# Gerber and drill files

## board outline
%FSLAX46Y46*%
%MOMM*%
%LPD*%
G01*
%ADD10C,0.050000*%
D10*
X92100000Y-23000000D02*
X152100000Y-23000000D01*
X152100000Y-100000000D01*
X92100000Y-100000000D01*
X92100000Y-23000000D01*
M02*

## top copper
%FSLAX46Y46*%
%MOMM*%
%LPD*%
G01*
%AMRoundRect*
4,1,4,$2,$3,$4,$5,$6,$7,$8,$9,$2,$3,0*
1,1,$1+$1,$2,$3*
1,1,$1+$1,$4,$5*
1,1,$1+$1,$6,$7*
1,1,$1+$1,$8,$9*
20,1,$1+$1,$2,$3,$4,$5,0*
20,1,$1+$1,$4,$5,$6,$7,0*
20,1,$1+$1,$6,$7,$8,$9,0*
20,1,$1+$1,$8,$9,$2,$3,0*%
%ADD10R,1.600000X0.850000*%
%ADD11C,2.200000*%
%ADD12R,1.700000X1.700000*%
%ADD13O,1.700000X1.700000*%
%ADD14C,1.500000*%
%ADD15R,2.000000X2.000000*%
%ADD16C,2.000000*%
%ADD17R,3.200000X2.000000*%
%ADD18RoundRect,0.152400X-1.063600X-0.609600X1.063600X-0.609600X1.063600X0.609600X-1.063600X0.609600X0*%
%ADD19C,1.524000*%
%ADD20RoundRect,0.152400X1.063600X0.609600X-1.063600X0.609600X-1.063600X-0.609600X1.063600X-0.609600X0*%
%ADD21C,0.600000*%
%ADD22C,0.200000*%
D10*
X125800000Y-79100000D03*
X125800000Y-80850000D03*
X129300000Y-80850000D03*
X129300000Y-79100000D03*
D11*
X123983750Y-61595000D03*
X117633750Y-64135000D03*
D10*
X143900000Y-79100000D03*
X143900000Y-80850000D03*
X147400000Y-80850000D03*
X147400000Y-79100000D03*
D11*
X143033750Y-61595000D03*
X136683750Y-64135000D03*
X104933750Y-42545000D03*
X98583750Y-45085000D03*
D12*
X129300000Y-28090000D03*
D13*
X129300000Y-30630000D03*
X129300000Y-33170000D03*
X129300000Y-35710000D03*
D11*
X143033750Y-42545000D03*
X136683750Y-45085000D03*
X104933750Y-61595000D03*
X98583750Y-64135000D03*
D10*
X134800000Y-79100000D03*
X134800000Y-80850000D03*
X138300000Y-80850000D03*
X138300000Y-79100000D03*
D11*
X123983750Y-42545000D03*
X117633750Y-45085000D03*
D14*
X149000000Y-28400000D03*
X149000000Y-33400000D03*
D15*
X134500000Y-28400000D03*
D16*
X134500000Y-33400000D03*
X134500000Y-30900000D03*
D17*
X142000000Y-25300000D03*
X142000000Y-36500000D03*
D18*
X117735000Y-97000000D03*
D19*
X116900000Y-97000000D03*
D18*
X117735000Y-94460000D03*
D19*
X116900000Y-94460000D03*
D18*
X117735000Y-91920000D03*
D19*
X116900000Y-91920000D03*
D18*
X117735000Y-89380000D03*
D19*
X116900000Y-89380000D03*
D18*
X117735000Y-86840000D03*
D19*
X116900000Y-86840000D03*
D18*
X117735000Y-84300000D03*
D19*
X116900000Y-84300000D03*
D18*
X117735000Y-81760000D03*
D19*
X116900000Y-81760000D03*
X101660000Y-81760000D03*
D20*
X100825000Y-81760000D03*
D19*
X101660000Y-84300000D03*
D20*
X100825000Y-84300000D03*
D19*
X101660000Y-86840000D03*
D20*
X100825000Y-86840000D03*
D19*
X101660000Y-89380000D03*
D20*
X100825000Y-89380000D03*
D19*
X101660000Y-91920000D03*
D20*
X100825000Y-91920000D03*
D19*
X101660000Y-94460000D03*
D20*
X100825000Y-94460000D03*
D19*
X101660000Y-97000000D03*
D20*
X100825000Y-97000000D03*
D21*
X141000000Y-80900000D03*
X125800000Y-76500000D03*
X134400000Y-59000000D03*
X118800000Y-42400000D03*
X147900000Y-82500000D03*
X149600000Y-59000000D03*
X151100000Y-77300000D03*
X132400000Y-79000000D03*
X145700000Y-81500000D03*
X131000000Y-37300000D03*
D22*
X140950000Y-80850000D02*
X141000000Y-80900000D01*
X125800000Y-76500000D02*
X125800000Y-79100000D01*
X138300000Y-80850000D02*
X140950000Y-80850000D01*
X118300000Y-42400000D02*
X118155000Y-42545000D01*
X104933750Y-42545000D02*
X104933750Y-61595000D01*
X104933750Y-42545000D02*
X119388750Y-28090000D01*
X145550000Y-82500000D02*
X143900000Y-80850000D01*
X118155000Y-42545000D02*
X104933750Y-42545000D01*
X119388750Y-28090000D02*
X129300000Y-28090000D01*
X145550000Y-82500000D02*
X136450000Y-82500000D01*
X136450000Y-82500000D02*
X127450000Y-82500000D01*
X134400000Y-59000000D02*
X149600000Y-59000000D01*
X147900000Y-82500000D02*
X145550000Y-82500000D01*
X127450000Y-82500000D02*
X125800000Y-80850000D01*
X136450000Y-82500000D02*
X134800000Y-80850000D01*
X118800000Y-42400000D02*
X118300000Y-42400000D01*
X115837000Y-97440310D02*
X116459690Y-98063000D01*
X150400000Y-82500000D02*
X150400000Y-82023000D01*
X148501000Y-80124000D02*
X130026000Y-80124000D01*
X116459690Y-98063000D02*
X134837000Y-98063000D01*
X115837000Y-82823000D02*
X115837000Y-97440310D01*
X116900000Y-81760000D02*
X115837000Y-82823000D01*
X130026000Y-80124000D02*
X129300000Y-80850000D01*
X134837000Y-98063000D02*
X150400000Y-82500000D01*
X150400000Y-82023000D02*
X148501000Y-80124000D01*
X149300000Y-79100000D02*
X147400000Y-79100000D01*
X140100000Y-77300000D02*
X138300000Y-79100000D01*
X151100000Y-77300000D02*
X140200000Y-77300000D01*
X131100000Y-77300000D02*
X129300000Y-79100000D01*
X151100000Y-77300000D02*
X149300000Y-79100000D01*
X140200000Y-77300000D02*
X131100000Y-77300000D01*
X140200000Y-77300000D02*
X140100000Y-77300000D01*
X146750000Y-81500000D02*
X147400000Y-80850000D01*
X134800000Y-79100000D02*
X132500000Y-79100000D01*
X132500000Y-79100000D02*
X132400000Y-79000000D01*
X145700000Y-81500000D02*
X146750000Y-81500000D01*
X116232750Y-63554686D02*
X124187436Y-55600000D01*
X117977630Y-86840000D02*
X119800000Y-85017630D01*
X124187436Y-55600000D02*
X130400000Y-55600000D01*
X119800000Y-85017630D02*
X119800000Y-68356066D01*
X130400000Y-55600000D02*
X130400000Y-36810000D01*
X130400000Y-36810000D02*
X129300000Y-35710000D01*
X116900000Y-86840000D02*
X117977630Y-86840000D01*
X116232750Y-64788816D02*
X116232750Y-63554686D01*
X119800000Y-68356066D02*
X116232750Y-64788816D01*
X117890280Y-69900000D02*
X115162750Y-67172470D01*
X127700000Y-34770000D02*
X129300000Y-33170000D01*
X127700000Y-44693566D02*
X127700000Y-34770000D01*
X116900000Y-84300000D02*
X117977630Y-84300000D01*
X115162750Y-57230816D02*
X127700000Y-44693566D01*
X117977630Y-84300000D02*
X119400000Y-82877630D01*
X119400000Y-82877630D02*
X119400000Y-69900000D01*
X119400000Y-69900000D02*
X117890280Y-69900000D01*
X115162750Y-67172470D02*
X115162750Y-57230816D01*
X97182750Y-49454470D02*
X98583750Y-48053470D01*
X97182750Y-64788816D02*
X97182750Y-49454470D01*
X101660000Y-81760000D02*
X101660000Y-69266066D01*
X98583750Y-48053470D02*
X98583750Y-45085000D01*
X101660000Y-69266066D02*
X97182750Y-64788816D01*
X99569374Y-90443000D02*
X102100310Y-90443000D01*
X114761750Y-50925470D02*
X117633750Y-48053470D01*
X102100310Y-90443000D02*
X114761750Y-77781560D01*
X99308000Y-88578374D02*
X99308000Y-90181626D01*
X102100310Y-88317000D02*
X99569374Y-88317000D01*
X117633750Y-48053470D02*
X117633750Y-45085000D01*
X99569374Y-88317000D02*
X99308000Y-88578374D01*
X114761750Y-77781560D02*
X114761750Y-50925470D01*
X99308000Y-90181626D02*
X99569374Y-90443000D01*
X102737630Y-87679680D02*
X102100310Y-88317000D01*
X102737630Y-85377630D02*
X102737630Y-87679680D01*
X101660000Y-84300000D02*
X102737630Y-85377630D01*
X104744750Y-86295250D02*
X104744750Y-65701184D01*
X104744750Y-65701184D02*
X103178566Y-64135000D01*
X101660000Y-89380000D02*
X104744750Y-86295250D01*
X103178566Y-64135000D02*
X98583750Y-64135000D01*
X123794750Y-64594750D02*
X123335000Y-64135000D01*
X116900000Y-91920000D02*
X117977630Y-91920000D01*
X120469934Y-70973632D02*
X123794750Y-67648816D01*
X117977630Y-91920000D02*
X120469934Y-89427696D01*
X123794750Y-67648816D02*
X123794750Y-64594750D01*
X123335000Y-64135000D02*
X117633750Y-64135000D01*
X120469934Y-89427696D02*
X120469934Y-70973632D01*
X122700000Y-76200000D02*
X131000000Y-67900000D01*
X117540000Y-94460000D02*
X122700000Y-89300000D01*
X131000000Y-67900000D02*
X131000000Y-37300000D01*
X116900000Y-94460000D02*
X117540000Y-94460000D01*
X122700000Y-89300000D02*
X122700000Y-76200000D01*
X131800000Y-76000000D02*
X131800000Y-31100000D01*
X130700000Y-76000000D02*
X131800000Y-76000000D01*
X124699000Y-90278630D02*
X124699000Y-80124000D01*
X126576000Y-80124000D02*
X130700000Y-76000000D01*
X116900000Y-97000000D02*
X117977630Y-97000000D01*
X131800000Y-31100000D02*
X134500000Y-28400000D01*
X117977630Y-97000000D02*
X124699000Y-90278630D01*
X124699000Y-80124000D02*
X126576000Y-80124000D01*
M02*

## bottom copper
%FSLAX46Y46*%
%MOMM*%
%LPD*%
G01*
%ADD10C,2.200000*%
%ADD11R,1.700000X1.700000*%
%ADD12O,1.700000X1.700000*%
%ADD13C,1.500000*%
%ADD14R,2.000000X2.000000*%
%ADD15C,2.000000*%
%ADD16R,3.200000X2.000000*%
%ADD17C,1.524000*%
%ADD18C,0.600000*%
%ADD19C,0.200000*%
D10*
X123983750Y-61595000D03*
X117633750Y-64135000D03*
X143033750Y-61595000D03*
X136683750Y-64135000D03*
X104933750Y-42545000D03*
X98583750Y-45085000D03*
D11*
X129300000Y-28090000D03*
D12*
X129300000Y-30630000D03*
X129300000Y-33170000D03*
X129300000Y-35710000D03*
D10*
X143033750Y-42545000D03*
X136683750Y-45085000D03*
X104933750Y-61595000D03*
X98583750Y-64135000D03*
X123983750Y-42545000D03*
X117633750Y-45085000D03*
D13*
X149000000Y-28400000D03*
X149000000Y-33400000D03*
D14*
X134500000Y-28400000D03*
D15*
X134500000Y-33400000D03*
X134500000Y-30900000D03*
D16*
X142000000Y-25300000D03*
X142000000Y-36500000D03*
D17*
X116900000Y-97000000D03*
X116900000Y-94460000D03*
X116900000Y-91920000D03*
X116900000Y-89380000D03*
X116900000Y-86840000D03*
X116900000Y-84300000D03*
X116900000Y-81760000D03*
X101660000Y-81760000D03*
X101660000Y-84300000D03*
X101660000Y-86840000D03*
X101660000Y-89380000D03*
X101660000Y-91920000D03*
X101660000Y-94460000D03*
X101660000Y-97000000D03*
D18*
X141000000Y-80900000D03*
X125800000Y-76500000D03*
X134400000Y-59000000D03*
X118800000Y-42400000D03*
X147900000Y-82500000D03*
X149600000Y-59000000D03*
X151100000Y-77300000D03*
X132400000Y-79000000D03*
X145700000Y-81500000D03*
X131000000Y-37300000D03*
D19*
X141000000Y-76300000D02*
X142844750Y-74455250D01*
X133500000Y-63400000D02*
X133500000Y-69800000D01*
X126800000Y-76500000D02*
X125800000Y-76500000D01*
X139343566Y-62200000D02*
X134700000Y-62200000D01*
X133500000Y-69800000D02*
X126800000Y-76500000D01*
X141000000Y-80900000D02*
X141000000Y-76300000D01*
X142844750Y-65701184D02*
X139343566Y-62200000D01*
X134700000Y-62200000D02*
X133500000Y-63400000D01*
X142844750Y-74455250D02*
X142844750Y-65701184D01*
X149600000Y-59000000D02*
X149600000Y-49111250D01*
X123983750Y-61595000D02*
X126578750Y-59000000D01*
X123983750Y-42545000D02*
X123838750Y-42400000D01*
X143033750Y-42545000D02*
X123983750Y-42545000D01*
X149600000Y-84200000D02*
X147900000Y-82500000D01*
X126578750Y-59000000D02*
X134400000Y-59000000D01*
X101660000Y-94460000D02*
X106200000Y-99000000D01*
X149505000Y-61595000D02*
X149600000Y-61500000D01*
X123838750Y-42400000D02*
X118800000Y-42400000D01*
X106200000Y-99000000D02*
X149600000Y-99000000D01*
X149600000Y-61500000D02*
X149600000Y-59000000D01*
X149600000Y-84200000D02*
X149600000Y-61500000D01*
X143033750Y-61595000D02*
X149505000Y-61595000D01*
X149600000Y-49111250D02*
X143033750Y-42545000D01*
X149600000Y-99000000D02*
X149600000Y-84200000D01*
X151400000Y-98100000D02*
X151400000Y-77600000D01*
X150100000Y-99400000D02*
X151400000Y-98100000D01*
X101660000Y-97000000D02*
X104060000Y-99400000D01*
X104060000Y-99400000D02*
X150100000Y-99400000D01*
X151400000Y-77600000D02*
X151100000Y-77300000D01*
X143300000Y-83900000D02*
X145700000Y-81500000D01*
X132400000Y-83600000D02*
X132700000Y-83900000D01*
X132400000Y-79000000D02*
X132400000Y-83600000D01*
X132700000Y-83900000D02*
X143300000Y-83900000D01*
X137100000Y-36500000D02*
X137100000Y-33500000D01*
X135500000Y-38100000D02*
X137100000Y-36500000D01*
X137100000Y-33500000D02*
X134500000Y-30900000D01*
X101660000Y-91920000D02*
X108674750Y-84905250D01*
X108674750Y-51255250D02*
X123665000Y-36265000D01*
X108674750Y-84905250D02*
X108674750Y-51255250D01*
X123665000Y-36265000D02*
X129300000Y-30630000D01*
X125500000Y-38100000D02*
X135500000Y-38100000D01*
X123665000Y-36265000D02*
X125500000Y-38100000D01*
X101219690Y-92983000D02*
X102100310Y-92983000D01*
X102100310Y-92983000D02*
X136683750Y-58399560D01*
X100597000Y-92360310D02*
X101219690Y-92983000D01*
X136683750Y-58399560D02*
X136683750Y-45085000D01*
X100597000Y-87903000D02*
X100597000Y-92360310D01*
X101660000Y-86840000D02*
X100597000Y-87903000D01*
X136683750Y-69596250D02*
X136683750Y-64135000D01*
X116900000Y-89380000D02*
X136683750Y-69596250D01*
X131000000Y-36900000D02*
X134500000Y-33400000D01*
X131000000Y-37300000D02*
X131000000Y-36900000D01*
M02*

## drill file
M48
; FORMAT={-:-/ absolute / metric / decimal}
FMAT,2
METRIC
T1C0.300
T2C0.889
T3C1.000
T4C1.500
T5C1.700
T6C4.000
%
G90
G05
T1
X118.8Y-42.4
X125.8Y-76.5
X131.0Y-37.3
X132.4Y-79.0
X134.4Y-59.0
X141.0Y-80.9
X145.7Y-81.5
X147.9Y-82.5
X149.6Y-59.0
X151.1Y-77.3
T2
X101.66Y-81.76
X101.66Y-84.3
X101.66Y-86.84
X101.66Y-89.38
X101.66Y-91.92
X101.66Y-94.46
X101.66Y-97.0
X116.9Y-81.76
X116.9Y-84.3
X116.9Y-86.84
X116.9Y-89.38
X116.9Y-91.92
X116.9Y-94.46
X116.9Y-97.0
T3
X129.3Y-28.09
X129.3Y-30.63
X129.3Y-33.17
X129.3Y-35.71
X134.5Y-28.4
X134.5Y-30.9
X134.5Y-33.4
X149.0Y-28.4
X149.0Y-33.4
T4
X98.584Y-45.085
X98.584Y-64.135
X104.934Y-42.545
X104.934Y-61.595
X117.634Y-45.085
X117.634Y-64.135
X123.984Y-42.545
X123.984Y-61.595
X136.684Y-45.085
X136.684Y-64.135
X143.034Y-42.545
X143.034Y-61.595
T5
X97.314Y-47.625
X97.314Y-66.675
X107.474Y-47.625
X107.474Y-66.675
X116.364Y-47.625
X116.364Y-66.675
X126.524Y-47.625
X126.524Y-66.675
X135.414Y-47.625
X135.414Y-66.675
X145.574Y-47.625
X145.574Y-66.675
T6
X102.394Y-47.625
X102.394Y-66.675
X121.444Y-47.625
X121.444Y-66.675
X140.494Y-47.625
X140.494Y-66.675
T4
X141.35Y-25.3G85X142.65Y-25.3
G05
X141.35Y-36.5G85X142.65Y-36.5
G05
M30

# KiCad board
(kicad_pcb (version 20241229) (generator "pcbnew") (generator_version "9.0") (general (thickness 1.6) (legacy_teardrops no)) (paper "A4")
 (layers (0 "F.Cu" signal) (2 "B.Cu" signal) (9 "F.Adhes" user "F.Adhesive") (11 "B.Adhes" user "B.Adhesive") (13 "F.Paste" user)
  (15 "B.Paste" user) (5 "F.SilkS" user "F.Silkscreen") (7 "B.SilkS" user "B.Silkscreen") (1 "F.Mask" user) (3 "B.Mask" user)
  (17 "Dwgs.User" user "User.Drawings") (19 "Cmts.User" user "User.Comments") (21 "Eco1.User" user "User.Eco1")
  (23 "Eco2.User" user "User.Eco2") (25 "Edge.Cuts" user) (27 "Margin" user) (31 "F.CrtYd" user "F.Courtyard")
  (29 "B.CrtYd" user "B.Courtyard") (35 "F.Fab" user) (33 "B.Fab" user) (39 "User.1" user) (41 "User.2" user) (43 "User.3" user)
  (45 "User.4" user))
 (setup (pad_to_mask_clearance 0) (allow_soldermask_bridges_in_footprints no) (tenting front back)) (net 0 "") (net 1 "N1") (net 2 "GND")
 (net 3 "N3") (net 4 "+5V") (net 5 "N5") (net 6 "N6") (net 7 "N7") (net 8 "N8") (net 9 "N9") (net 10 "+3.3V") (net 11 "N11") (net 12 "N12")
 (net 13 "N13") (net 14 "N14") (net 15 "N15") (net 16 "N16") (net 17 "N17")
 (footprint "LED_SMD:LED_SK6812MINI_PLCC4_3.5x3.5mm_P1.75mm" (layer "F.Cu") (at 127.55 79.975)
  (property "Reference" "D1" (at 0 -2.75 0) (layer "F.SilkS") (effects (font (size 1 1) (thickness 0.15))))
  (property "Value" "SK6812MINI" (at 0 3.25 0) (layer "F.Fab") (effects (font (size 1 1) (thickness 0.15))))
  (pad "1" smd rect (at -1.75 -0.875) (size 1.6 0.85) (layers "F.Cu" "F.Mask" "F.Paste") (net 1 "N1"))
  (pad "2" smd rect (at -1.75 0.875) (size 1.6 0.85) (layers "F.Cu" "F.Mask" "F.Paste") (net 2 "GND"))
  (pad "3" smd rect (at 1.75 0.875) (size 1.6 0.85) (layers "F.Cu" "F.Mask" "F.Paste") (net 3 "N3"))
  (pad "4" smd rect (at 1.75 -0.875) (size 1.6 0.85) (layers "F.Cu" "F.Mask" "F.Paste") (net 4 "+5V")))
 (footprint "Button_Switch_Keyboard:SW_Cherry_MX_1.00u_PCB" (layer "F.Cu") (at 123.98375 61.595)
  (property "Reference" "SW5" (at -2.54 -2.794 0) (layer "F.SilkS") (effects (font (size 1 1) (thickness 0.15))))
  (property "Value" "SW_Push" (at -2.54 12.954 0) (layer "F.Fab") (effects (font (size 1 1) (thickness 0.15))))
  (pad "" np_thru_hole circle (at -7.62 5.08) (size 1.7 1.7) (drill 1.7) (layers "*.Cu" "*.Mask"))
  (pad "" np_thru_hole circle (at -2.54 5.08) (size 4 4) (drill 4) (layers "*.Cu" "*.Mask"))
  (pad "" np_thru_hole circle (at 2.54 5.08) (size 1.7 1.7) (drill 1.7) (layers "*.Cu" "*.Mask"))
  (pad "1" thru_hole circle (at 0 0) (size 2.2 2.2) (drill 1.5) (layers "*.Cu" "*.Mask") (remove_unused_layers no) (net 2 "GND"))
  (pad "2" thru_hole circle (at -6.35 2.54) (size 2.2 2.2) (drill 1.5) (layers "*.Cu" "*.Mask") (remove_unused_layers no) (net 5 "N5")))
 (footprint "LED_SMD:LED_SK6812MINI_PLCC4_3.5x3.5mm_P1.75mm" (layer "F.Cu") (at 145.65 79.975)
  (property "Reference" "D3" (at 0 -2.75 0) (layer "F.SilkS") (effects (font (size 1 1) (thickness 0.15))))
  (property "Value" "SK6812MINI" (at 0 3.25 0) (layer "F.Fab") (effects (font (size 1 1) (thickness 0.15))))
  (pad "1" smd rect (at -1.75 -0.875) (size 1.6 0.85) (layers "F.Cu" "F.Mask" "F.Paste") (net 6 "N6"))
  (pad "2" smd rect (at -1.75 0.875) (size 1.6 0.85) (layers "F.Cu" "F.Mask" "F.Paste") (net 2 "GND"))
  (pad "3" smd rect (at 1.75 0.875) (size 1.6 0.85) (layers "F.Cu" "F.Mask" "F.Paste") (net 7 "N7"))
  (pad "4" smd rect (at 1.75 -0.875) (size 1.6 0.85) (layers "F.Cu" "F.Mask" "F.Paste") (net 4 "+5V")))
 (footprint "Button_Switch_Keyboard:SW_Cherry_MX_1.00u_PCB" (layer "F.Cu") (at 143.03375 61.595)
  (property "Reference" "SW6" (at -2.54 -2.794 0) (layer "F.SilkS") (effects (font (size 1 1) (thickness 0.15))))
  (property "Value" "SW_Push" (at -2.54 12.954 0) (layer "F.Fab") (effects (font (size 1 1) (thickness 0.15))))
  (pad "" np_thru_hole circle (at -7.62 5.08) (size 1.7 1.7) (drill 1.7) (layers "*.Cu" "*.Mask"))
  (pad "" np_thru_hole circle (at -2.54 5.08) (size 4 4) (drill 4) (layers "*.Cu" "*.Mask"))
  (pad "" np_thru_hole circle (at 2.54 5.08) (size 1.7 1.7) (drill 1.7) (layers "*.Cu" "*.Mask"))
  (pad "1" thru_hole circle (at 0 0) (size 2.2 2.2) (drill 1.5) (layers "*.Cu" "*.Mask") (remove_unused_layers no) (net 2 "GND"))
  (pad "2" thru_hole circle (at -6.35 2.54) (size 2.2 2.2) (drill 1.5) (layers "*.Cu" "*.Mask") (remove_unused_layers no) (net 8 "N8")))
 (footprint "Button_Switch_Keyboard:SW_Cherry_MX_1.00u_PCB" (layer "F.Cu") (at 104.93375 42.545)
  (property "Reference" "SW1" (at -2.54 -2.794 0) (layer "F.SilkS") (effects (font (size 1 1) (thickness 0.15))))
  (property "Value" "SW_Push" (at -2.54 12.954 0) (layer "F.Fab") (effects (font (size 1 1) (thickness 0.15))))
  (pad "" np_thru_hole circle (at -7.62 5.08) (size 1.7 1.7) (drill 1.7) (layers "*.Cu" "*.Mask"))
  (pad "" np_thru_hole circle (at -2.54 5.08) (size 4 4) (drill 4) (layers "*.Cu" "*.Mask"))
  (pad "" np_thru_hole circle (at 2.54 5.08) (size 1.7 1.7) (drill 1.7) (layers "*.Cu" "*.Mask"))
  (pad "1" thru_hole circle (at 0 0) (size 2.2 2.2) (drill 1.5) (layers "*.Cu" "*.Mask") (remove_unused_layers no) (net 2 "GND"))
  (pad "2" thru_hole circle (at -6.35 2.54) (size 2.2 2.2) (drill 1.5) (layers "*.Cu" "*.Mask") (remove_unused_layers no) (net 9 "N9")))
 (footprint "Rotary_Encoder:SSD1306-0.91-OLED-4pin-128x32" (layer "F.Cu") (at 92.8 25.9)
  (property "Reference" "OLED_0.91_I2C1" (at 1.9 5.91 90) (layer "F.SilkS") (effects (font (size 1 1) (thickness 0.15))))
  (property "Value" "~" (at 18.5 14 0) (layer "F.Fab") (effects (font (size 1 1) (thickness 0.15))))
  (pad "1" thru_hole rect (at 36.5 2.19) (size 1.7 1.7) (drill 1) (layers "*.Cu" "*.Mask") (remove_unused_layers no) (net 2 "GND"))
  (pad "2" thru_hole oval (at 36.5 4.73) (size 1.7 1.7) (drill 1) (layers "*.Cu" "*.Mask") (remove_unused_layers no) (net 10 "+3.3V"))
  (pad "3" thru_hole oval (at 36.5 7.27) (size 1.7 1.7) (drill 1) (layers "*.Cu" "*.Mask") (remove_unused_layers no) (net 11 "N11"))
  (pad "4" thru_hole oval (at 36.5 9.81) (size 1.7 1.7) (drill 1) (layers "*.Cu" "*.Mask") (remove_unused_layers no) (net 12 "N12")))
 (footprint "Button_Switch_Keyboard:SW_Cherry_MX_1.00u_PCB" (layer "F.Cu") (at 143.03375 42.545)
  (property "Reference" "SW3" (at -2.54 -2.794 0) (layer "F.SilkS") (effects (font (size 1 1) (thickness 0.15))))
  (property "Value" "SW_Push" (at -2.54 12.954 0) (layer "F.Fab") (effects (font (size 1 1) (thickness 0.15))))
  (pad "" np_thru_hole circle (at -7.62 5.08) (size 1.7 1.7) (drill 1.7) (layers "*.Cu" "*.Mask"))
  (pad "" np_thru_hole circle (at -2.54 5.08) (size 4 4) (drill 4) (layers "*.Cu" "*.Mask"))
  (pad "" np_thru_hole circle (at 2.54 5.08) (size 1.7 1.7) (drill 1.7) (layers "*.Cu" "*.Mask"))
  (pad "1" thru_hole circle (at 0 0) (size 2.2 2.2) (drill 1.5) (layers "*.Cu" "*.Mask") (remove_unused_layers no) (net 2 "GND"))
  (pad "2" thru_hole circle (at -6.35 2.54) (size 2.2 2.2) (drill 1.5) (layers "*.Cu" "*.Mask") (remove_unused_layers no) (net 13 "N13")))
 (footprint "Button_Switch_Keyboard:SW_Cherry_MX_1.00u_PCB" (layer "F.Cu") (at 104.93375 61.595)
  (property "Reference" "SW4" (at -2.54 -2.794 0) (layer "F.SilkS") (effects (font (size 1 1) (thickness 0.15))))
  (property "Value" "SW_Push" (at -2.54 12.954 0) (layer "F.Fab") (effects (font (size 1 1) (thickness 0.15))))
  (pad "" np_thru_hole circle (at -7.62 5.08) (size 1.7 1.7) (drill 1.7) (layers "*.Cu" "*.Mask"))
  (pad "" np_thru_hole circle (at -2.54 5.08) (size 4 4) (drill 4) (layers "*.Cu" "*.Mask"))
  (pad "" np_thru_hole circle (at 2.54 5.08) (size 1.7 1.7) (drill 1.7) (layers "*.Cu" "*.Mask"))
  (pad "1" thru_hole circle (at 0 0) (size 2.2 2.2) (drill 1.5) (layers "*.Cu" "*.Mask") (remove_unused_layers no) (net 2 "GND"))
  (pad "2" thru_hole circle (at -6.35 2.54) (size 2.2 2.2) (drill 1.5) (layers "*.Cu" "*.Mask") (remove_unused_layers no) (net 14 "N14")))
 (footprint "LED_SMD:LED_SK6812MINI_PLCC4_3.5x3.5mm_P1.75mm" (layer "F.Cu") (at 136.55 79.975)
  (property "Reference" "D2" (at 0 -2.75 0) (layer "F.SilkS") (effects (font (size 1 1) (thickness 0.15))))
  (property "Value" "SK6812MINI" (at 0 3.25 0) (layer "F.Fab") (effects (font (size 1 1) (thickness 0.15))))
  (pad "1" smd rect (at -1.75 -0.875) (size 1.6 0.85) (layers "F.Cu" "F.Mask" "F.Paste") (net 7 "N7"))
  (pad "2" smd rect (at -1.75 0.875) (size 1.6 0.85) (layers "F.Cu" "F.Mask" "F.Paste") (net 2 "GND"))
  (pad "3" smd rect (at 1.75 0.875) (size 1.6 0.85) (layers "F.Cu" "F.Mask" "F.Paste") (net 1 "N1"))
  (pad "4" smd rect (at 1.75 -0.875) (size 1.6 0.85) (layers "F.Cu" "F.Mask" "F.Paste") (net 4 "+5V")))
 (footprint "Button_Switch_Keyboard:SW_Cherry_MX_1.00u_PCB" (layer "F.Cu") (at 123.98375 42.545)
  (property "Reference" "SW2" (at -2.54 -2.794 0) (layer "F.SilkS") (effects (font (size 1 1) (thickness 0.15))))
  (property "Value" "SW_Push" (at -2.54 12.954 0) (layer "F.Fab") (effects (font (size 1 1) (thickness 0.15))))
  (pad "" np_thru_hole circle (at -7.62 5.08) (size 1.7 1.7) (drill 1.7) (layers "*.Cu" "*.Mask"))
  (pad "" np_thru_hole circle (at -2.54 5.08) (size 4 4) (drill 4) (layers "*.Cu" "*.Mask"))
  (pad "" np_thru_hole circle (at 2.54 5.08) (size 1.7 1.7) (drill 1.7) (layers "*.Cu" "*.Mask"))
  (pad "1" thru_hole circle (at 0 0) (size 2.2 2.2) (drill 1.5) (layers "*.Cu" "*.Mask") (remove_unused_layers no) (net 2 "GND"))
  (pad "2" thru_hole circle (at -6.35 2.54) (size 2.2 2.2) (drill 1.5) (layers "*.Cu" "*.Mask") (remove_unused_layers no) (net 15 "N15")))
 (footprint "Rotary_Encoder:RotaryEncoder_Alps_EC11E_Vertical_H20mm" (layer "F.Cu") (at 134.5 28.4)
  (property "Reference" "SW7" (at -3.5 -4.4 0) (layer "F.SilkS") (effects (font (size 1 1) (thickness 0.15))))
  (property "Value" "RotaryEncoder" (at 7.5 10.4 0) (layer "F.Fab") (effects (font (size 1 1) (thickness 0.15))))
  (pad "" thru_hole circle (at 14.5 0) (size 1.5 1.5) (drill 1) (layers "*.Cu" "*.Mask") (remove_unused_layers no))
  (pad "" thru_hole circle (at 14.5 5) (size 1.5 1.5) (drill 1) (layers "*.Cu" "*.Mask") (remove_unused_layers no))
  (pad "A" thru_hole rect (at 0 0) (size 2 2) (drill 1) (layers "*.Cu" "*.Mask") (remove_unused_layers no) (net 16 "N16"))
  (pad "B" thru_hole circle (at 0 5) (size 2 2) (drill 1) (layers "*.Cu" "*.Mask") (remove_unused_layers no) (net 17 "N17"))
  (pad "C" thru_hole circle (at 0 2.5) (size 2 2) (drill 1) (layers "*.Cu" "*.Mask") (remove_unused_layers no) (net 10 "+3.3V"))
  (pad "MP" thru_hole rect (at 7.5 -3.1) (size 3.2 2) (drill oval 2.8 1.5) (layers "*.Cu" "*.Mask") (remove_unused_layers no))
  (pad "MP" thru_hole rect (at 7.5 8.1) (size 3.2 2) (drill oval 2.8 1.5) (layers "*.Cu" "*.Mask") (remove_unused_layers no)))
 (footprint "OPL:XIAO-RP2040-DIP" (layer "F.Cu") (at 109.28 89.38 180)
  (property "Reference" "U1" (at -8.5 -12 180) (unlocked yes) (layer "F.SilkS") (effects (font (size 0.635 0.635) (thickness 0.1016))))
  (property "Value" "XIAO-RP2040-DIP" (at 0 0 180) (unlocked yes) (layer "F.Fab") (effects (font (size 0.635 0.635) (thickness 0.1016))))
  (pad "1" smd roundrect (at -8.455 -7.62) (size 2.432 1.524) (layers "F.Cu" "F.Mask") (roundrect_rratio 0.1) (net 16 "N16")
   (thermal_bridge_angle 45))
  (pad "1" thru_hole circle (at -7.62 -7.62) (size 1.524 1.524) (drill 0.889) (layers "*.Cu" "*.Mask") (remove_unused_layers no)
   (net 16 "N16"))
  (pad "2" smd roundrect (at -8.455 -5.08) (size 2.432 1.524) (layers "F.Cu" "F.Mask") (roundrect_rratio 0.1) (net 17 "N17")
   (thermal_bridge_angle 45))
  (pad "2" thru_hole circle (at -7.62 -5.08) (size 1.524 1.524) (drill 0.889) (layers "*.Cu" "*.Mask") (remove_unused_layers no)
   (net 17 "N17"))
  (pad "3" smd roundrect (at -8.455 -2.54) (size 2.432 1.524) (layers "F.Cu" "F.Mask") (roundrect_rratio 0.1) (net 5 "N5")
   (thermal_bridge_angle 45))
  (pad "3" thru_hole circle (at -7.62 -2.54) (size 1.524 1.524) (drill 0.889) (layers "*.Cu" "*.Mask") (remove_unused_layers no)
   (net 5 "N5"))
  (pad "4" smd roundrect (at -8.455 0) (size 2.432 1.524) (layers "F.Cu" "F.Mask") (roundrect_rratio 0.1) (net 8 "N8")
   (thermal_bridge_angle 45))
  (pad "4" thru_hole circle (at -7.62 0) (size 1.524 1.524) (drill 0.889) (layers "*.Cu" "*.Mask") (remove_unused_layers no) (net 8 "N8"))
  (pad "5" smd roundrect (at -8.455 2.54) (size 2.432 1.524) (layers "F.Cu" "F.Mask") (roundrect_rratio 0.1) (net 12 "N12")
   (thermal_bridge_angle 45))
  (pad "5" thru_hole circle (at -7.62 2.54) (size 1.524 1.524) (drill 0.889) (layers "*.Cu" "*.Mask") (remove_unused_layers no)
   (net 12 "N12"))
  (pad "6" smd roundrect (at -8.455 5.08) (size 2.432 1.524) (layers "F.Cu" "F.Mask") (roundrect_rratio 0.1) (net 11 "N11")
   (thermal_bridge_angle 45))
  (pad "6" thru_hole circle (at -7.62 5.08) (size 1.524 1.524) (drill 0.889) (layers "*.Cu" "*.Mask") (remove_unused_layers no)
   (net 11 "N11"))
  (pad "7" smd roundrect (at -8.455 7.62) (size 2.432 1.524) (layers "F.Cu" "F.Mask") (roundrect_rratio 0.1) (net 3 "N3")
   (thermal_bridge_angle 45))
  (pad "7" thru_hole circle (at -7.62 7.62) (size 1.524 1.524) (drill 0.889) (layers "*.Cu" "*.Mask") (remove_unused_layers no) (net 3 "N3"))
  (pad "8" thru_hole circle (at 7.62 7.62 180) (size 1.524 1.524) (drill 0.889) (layers "*.Cu" "*.Mask") (remove_unused_layers no)
   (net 9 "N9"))
  (pad "8" smd roundrect (at 8.455 7.62 180) (size 2.432 1.524) (layers "F.Cu" "F.Mask") (roundrect_rratio 0.1) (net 9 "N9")
   (thermal_bridge_angle 45))
  (pad "9" thru_hole circle (at 7.62 5.08 180) (size 1.524 1.524) (drill 0.889) (layers "*.Cu" "*.Mask") (remove_unused_layers no)
   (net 15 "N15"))
  (pad "9" smd roundrect (at 8.455 5.08 180) (size 2.432 1.524) (layers "F.Cu" "F.Mask") (roundrect_rratio 0.1) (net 15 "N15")
   (thermal_bridge_angle 45))
  (pad "10" thru_hole circle (at 7.62 2.54 180) (size 1.524 1.524) (drill 0.889) (layers "*.Cu" "*.Mask") (remove_unused_layers no)
   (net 13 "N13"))
  (pad "10" smd roundrect (at 8.455 2.54 180) (size 2.432 1.524) (layers "F.Cu" "F.Mask") (roundrect_rratio 0.1) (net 13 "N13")
   (thermal_bridge_angle 45))
  (pad "11" thru_hole circle (at 7.62 0 180) (size 1.524 1.524) (drill 0.889) (layers "*.Cu" "*.Mask") (remove_unused_layers no)
   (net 14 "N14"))
  (pad "11" smd roundrect (at 8.455 0 180) (size 2.432 1.524) (layers "F.Cu" "F.Mask") (roundrect_rratio 0.1) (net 14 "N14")
   (thermal_bridge_angle 45))
  (pad "12" thru_hole circle (at 7.62 -2.54 180) (size 1.524 1.524) (drill 0.889) (layers "*.Cu" "*.Mask") (remove_unused_layers no)
   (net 10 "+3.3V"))
  (pad "12" smd roundrect (at 8.455 -2.54 180) (size 2.432 1.524) (layers "F.Cu" "F.Mask") (roundrect_rratio 0.1) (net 10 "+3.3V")
   (thermal_bridge_angle 45))
  (pad "13" thru_hole circle (at 7.62 -5.08 180) (size 1.524 1.524) (drill 0.889) (layers "*.Cu" "*.Mask") (remove_unused_layers no)
   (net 2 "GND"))
  (pad "13" smd roundrect (at 8.455 -5.08 180) (size 2.432 1.524) (layers "F.Cu" "F.Mask") (roundrect_rratio 0.1) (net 2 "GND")
   (thermal_bridge_angle 45))
  (pad "14" thru_hole circle (at 7.62 -7.62 180) (size 1.524 1.524) (drill 0.889) (layers "*.Cu" "*.Mask") (remove_unused_layers no)
   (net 4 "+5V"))
  (pad "14" smd roundrect (at 8.455 -7.62 180) (size 2.432 1.524) (layers "F.Cu" "F.Mask") (roundrect_rratio 0.1) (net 4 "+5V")
   (thermal_bridge_angle 45)))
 (gr_rect (start 92.1 23) (end 152.1 100) (stroke (width 0.05) (type default)) (fill no) (layer "Edge.Cuts"))
 (segment (start 140.95 80.85) (end 141 80.9) (width 0.2) (layer "F.Cu") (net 1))
 (segment (start 125.8 76.5) (end 125.8 79.1) (width 0.2) (layer "F.Cu") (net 1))
 (segment (start 138.3 80.85) (end 140.95 80.85) (width 0.2) (layer "F.Cu") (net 1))
 (via (at 141 80.9) (size 0.6) (drill 0.3) (layers "F.Cu" "B.Cu") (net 1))
 (via (at 125.8 76.5) (size 0.6) (drill 0.3) (layers "F.Cu" "B.Cu") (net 1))
 (segment (start 141 76.3) (end 142.84475 74.45525) (width 0.2) (layer "B.Cu") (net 1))
 (segment (start 133.5 63.4) (end 133.5 69.8) (width 0.2) (layer "B.Cu") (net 1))
 (segment (start 126.8 76.5) (end 125.8 76.5) (width 0.2) (layer "B.Cu") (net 1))
 (segment (start 139.343566 62.2) (end 134.7 62.2) (width 0.2) (layer "B.Cu") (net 1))
 (segment (start 133.5 69.8) (end 126.8 76.5) (width 0.2) (layer "B.Cu") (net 1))
 (segment (start 141 80.9) (end 141 76.3) (width 0.2) (layer "B.Cu") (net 1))
 (segment (start 142.84475 65.701184) (end 139.343566 62.2) (width 0.2) (layer "B.Cu") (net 1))
 (segment (start 134.7 62.2) (end 133.5 63.4) (width 0.2) (layer "B.Cu") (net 1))
 (segment (start 142.84475 74.45525) (end 142.84475 65.701184) (width 0.2) (layer "B.Cu") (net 1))
 (segment (start 118.3 42.4) (end 118.155 42.545) (width 0.2) (layer "F.Cu") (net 2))
 (segment (start 104.93375 42.545) (end 104.93375 61.595) (width 0.2) (layer "F.Cu") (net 2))
 (segment (start 104.93375 42.545) (end 119.38875 28.09) (width 0.2) (layer "F.Cu") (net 2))
 (segment (start 145.55 82.5) (end 143.9 80.85) (width 0.2) (layer "F.Cu") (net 2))
 (segment (start 118.155 42.545) (end 104.93375 42.545) (width 0.2) (layer "F.Cu") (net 2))
 (segment (start 119.38875 28.09) (end 129.3 28.09) (width 0.2) (layer "F.Cu") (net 2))
 (segment (start 145.55 82.5) (end 136.45 82.5) (width 0.2) (layer "F.Cu") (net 2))
 (segment (start 136.45 82.5) (end 127.45 82.5) (width 0.2) (layer "F.Cu") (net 2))
 (segment (start 134.4 59) (end 149.6 59) (width 0.2) (layer "F.Cu") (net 2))
 (segment (start 147.9 82.5) (end 145.55 82.5) (width 0.2) (layer "F.Cu") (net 2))
 (segment (start 127.45 82.5) (end 125.8 80.85) (width 0.2) (layer "F.Cu") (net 2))
 (segment (start 136.45 82.5) (end 134.8 80.85) (width 0.2) (layer "F.Cu") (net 2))
 (segment (start 118.8 42.4) (end 118.3 42.4) (width 0.2) (layer "F.Cu") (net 2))
 (via (at 134.4 59) (size 0.6) (drill 0.3) (layers "F.Cu" "B.Cu") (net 2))
 (via (at 118.8 42.4) (size 0.6) (drill 0.3) (layers "F.Cu" "B.Cu") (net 2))
 (via (at 147.9 82.5) (size 0.6) (drill 0.3) (layers "F.Cu" "B.Cu") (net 2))
 (via (at 149.6 59) (size 0.6) (drill 0.3) (layers "F.Cu" "B.Cu") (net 2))
 (segment (start 149.6 59) (end 149.6 49.11125) (width 0.2) (layer "B.Cu") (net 2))
 (segment (start 123.98375 61.595) (end 126.57875 59) (width 0.2) (layer "B.Cu") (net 2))
 (segment (start 123.98375 42.545) (end 123.83875 42.4) (width 0.2) (layer "B.Cu") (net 2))
 (segment (start 143.03375 42.545) (end 123.98375 42.545) (width 0.2) (layer "B.Cu") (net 2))
 (segment (start 149.6 84.2) (end 147.9 82.5) (width 0.2) (layer "B.Cu") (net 2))
 (segment (start 126.57875 59) (end 134.4 59) (width 0.2) (layer "B.Cu") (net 2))
 (segment (start 101.66 94.46) (end 106.2 99) (width 0.2) (layer "B.Cu") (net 2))
 (segment (start 149.505 61.595) (end 149.6 61.5) (width 0.2) (layer "B.Cu") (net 2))
 (segment (start 123.83875 42.4) (end 118.8 42.4) (width 0.2) (layer "B.Cu") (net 2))
 (segment (start 106.2 99) (end 149.6 99) (width 0.2) (layer "B.Cu") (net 2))
 (segment (start 149.6 61.5) (end 149.6 59) (width 0.2) (layer "B.Cu") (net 2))
 (segment (start 149.6 84.2) (end 149.6 61.5) (width 0.2) (layer "B.Cu") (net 2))
 (segment (start 143.03375 61.595) (end 149.505 61.595) (width 0.2) (layer "B.Cu") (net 2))
 (segment (start 149.6 49.11125) (end 143.03375 42.545) (width 0.2) (layer "B.Cu") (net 2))
 (segment (start 149.6 99) (end 149.6 84.2) (width 0.2) (layer "B.Cu") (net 2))
 (segment (start 115.837 97.44031) (end 116.45969 98.063) (width 0.2) (layer "F.Cu") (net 3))
 (segment (start 150.4 82.5) (end 150.4 82.023) (width 0.2) (layer "F.Cu") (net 3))
 (segment (start 148.501 80.124) (end 130.026 80.124) (width 0.2) (layer "F.Cu") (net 3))
 (segment (start 116.45969 98.063) (end 134.837 98.063) (width 0.2) (layer "F.Cu") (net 3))
 (segment (start 115.837 82.823) (end 115.837 97.44031) (width 0.2) (layer "F.Cu") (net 3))
 (segment (start 116.9 81.76) (end 115.837 82.823) (width 0.2) (layer "F.Cu") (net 3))
 (segment (start 130.026 80.124) (end 129.3 80.85) (width 0.2) (layer "F.Cu") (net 3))
 (segment (start 134.837 98.063) (end 150.4 82.5) (width 0.2) (layer "F.Cu") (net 3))
 (segment (start 150.4 82.023) (end 148.501 80.124) (width 0.2) (layer "F.Cu") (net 3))
 (segment (start 149.3 79.1) (end 147.4 79.1) (width 0.2) (layer "F.Cu") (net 4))
 (segment (start 140.1 77.3) (end 138.3 79.1) (width 0.2) (layer "F.Cu") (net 4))
 (segment (start 151.1 77.3) (end 140.2 77.3) (width 0.2) (layer "F.Cu") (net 4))
 (segment (start 131.1 77.3) (end 129.3 79.1) (width 0.2) (layer "F.Cu") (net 4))
 (segment (start 151.1 77.3) (end 149.3 79.1) (width 0.2) (layer "F.Cu") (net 4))
 (segment (start 140.2 77.3) (end 131.1 77.3) (width 0.2) (layer "F.Cu") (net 4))
 (segment (start 140.2 77.3) (end 140.1 77.3) (width 0.2) (layer "F.Cu") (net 4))
 (via (at 151.1 77.3) (size 0.6) (drill 0.3) (layers "F.Cu" "B.Cu") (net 4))
 (segment (start 151.4 98.1) (end 151.4 77.6) (width 0.2) (layer "B.Cu") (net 4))
 (segment (start 150.1 99.4) (end 151.4 98.1) (width 0.2) (layer "B.Cu") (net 4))
 (segment (start 101.66 97) (end 104.06 99.4) (width 0.2) (layer "B.Cu") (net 4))
 (segment (start 104.06 99.4) (end 150.1 99.4) (width 0.2) (layer "B.Cu") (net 4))
 (segment (start 151.4 77.6) (end 151.1 77.3) (width 0.2) (layer "B.Cu") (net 4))
 (segment (start 146.75 81.5) (end 147.4 80.85) (width 0.2) (layer "F.Cu") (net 7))
 (segment (start 134.8 79.1) (end 132.5 79.1) (width 0.2) (layer "F.Cu") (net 7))
 (segment (start 132.5 79.1) (end 132.4 79) (width 0.2) (layer "F.Cu") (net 7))
 (segment (start 145.7 81.5) (end 146.75 81.5) (width 0.2) (layer "F.Cu") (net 7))
 (via (at 132.4 79) (size 0.6) (drill 0.3) (layers "F.Cu" "B.Cu") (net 7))
 (via (at 145.7 81.5) (size 0.6) (drill 0.3) (layers "F.Cu" "B.Cu") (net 7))
 (segment (start 143.3 83.9) (end 145.7 81.5) (width 0.2) (layer "B.Cu") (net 7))
 (segment (start 132.4 83.6) (end 132.7 83.9) (width 0.2) (layer "B.Cu") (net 7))
 (segment (start 132.4 79) (end 132.4 83.6) (width 0.2) (layer "B.Cu") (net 7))
 (segment (start 132.7 83.9) (end 143.3 83.9) (width 0.2) (layer "B.Cu") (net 7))
 (segment (start 137.1 36.5) (end 137.1 33.5) (width 0.2) (layer "B.Cu") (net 10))
 (segment (start 135.5 38.1) (end 137.1 36.5) (width 0.2) (layer "B.Cu") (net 10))
 (segment (start 137.1 33.5) (end 134.5 30.9) (width 0.2) (layer "B.Cu") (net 10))
 (segment (start 101.66 91.92) (end 108.67475 84.90525) (width 0.2) (layer "B.Cu") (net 10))
 (segment (start 108.67475 51.25525) (end 123.665 36.265) (width 0.2) (layer "B.Cu") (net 10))
 (segment (start 108.67475 84.90525) (end 108.67475 51.25525) (width 0.2) (layer "B.Cu") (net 10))
 (segment (start 123.665 36.265) (end 129.3 30.63) (width 0.2) (layer "B.Cu") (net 10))
 (segment (start 125.5 38.1) (end 135.5 38.1) (width 0.2) (layer "B.Cu") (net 10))
 (segment (start 123.665 36.265) (end 125.5 38.1) (width 0.2) (layer "B.Cu") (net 10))
 (segment (start 116.23275 63.554686) (end 124.187436 55.6) (width 0.2) (layer "F.Cu") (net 12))
 (segment (start 117.97763 86.84) (end 119.8 85.01763) (width 0.2) (layer "F.Cu") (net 12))
 (segment (start 124.187436 55.6) (end 130.4 55.6) (width 0.2) (layer "F.Cu") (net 12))
 (segment (start 119.8 85.01763) (end 119.8 68.356066) (width 0.2) (layer "F.Cu") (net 12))
 (segment (start 130.4 55.6) (end 130.4 36.81) (width 0.2) (layer "F.Cu") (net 12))
 (segment (start 130.4 36.81) (end 129.3 35.71) (width 0.2) (layer "F.Cu") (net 12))
 (segment (start 116.9 86.84) (end 117.97763 86.84) (width 0.2) (layer "F.Cu") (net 12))
 (segment (start 116.23275 64.788816) (end 116.23275 63.554686) (width 0.2) (layer "F.Cu") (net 12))
 (segment (start 119.8 68.356066) (end 116.23275 64.788816) (width 0.2) (layer "F.Cu") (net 12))
 (segment (start 117.89028 69.9) (end 115.16275 67.17247) (width 0.2) (layer "F.Cu") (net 11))
 (segment (start 127.7 34.77) (end 129.3 33.17) (width 0.2) (layer "F.Cu") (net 11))
 (segment (start 127.7 44.693566) (end 127.7 34.77) (width 0.2) (layer "F.Cu") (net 11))
 (segment (start 116.9 84.3) (end 117.97763 84.3) (width 0.2) (layer "F.Cu") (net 11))
 (segment (start 115.16275 57.230816) (end 127.7 44.693566) (width 0.2) (layer "F.Cu") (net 11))
 (segment (start 117.97763 84.3) (end 119.4 82.87763) (width 0.2) (layer "F.Cu") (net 11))
 (segment (start 119.4 82.87763) (end 119.4 69.9) (width 0.2) (layer "F.Cu") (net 11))
 (segment (start 119.4 69.9) (end 117.89028 69.9) (width 0.2) (layer "F.Cu") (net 11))
 (segment (start 115.16275 67.17247) (end 115.16275 57.230816) (width 0.2) (layer "F.Cu") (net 11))
 (segment (start 97.18275 49.45447) (end 98.58375 48.05347) (width 0.2) (layer "F.Cu") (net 9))
 (segment (start 97.18275 64.788816) (end 97.18275 49.45447) (width 0.2) (layer "F.Cu") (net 9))
 (segment (start 101.66 81.76) (end 101.66 69.266066) (width 0.2) (layer "F.Cu") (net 9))
 (segment (start 98.58375 48.05347) (end 98.58375 45.085) (width 0.2) (layer "F.Cu") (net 9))
 (segment (start 101.66 69.266066) (end 97.18275 64.788816) (width 0.2) (layer "F.Cu") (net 9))
 (segment (start 99.569374 90.443) (end 102.10031 90.443) (width 0.2) (layer "F.Cu") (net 15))
 (segment (start 114.76175 50.92547) (end 117.63375 48.05347) (width 0.2) (layer "F.Cu") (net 15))
 (segment (start 102.10031 90.443) (end 114.76175 77.78156) (width 0.2) (layer "F.Cu") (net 15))
 (segment (start 99.308 88.578374) (end 99.308 90.181626) (width 0.2) (layer "F.Cu") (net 15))
 (segment (start 102.10031 88.317) (end 99.569374 88.317) (width 0.2) (layer "F.Cu") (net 15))
 (segment (start 117.63375 48.05347) (end 117.63375 45.085) (width 0.2) (layer "F.Cu") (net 15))
 (segment (start 99.569374 88.317) (end 99.308 88.578374) (width 0.2) (layer "F.Cu") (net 15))
 (segment (start 114.76175 77.78156) (end 114.76175 50.92547) (width 0.2) (layer "F.Cu") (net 15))
 (segment (start 99.308 90.181626) (end 99.569374 90.443) (width 0.2) (layer "F.Cu") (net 15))
 (segment (start 102.73763 87.67968) (end 102.10031 88.317) (width 0.2) (layer "F.Cu") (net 15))
 (segment (start 102.73763 85.37763) (end 102.73763 87.67968) (width 0.2) (layer "F.Cu") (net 15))
 (segment (start 101.66 84.3) (end 102.73763 85.37763) (width 0.2) (layer "F.Cu") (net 15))
 (segment (start 101.21969 92.983) (end 102.10031 92.983) (width 0.2) (layer "B.Cu") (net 13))
 (segment (start 102.10031 92.983) (end 136.68375 58.39956) (width 0.2) (layer "B.Cu") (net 13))
 (segment (start 100.597 92.36031) (end 101.21969 92.983) (width 0.2) (layer "B.Cu") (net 13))
 (segment (start 136.68375 58.39956) (end 136.68375 45.085) (width 0.2) (layer "B.Cu") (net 13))
 (segment (start 100.597 87.903) (end 100.597 92.36031) (width 0.2) (layer "B.Cu") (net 13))
 (segment (start 101.66 86.84) (end 100.597 87.903) (width 0.2) (layer "B.Cu") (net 13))
 (segment (start 104.74475 86.29525) (end 104.74475 65.701184) (width 0.2) (layer "F.Cu") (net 14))
 (segment (start 104.74475 65.701184) (end 103.178566 64.135) (width 0.2) (layer "F.Cu") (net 14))
 (segment (start 101.66 89.38) (end 104.74475 86.29525) (width 0.2) (layer "F.Cu") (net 14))
 (segment (start 103.178566 64.135) (end 98.58375 64.135) (width 0.2) (layer "F.Cu") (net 14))
 (segment (start 123.79475 64.59475) (end 123.335 64.135) (width 0.2) (layer "F.Cu") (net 5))
 (segment (start 116.9 91.92) (end 117.97763 91.92) (width 0.2) (layer "F.Cu") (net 5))
 (segment (start 120.469934 70.973632) (end 123.79475 67.648816) (width 0.2) (layer "F.Cu") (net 5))
 (segment (start 117.97763 91.92) (end 120.469934 89.427696) (width 0.2) (layer "F.Cu") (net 5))
 (segment (start 123.79475 67.648816) (end 123.79475 64.59475) (width 0.2) (layer "F.Cu") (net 5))
 (segment (start 123.335 64.135) (end 117.63375 64.135) (width 0.2) (layer "F.Cu") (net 5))
 (segment (start 120.469934 89.427696) (end 120.469934 70.973632) (width 0.2) (layer "F.Cu") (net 5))
 (segment (start 136.68375 69.59625) (end 136.68375 64.135) (width 0.2) (layer "B.Cu") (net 8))
 (segment (start 116.9 89.38) (end 136.68375 69.59625) (width 0.2) (layer "B.Cu") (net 8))
 (segment (start 122.7 76.2) (end 131 67.9) (width 0.2) (layer "F.Cu") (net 17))
 (segment (start 117.54 94.46) (end 122.7 89.3) (width 0.2) (layer "F.Cu") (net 17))
 (segment (start 131 67.9) (end 131 37.3) (width 0.2) (layer "F.Cu") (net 17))
 (segment (start 116.9 94.46) (end 117.54 94.46) (width 0.2) (layer "F.Cu") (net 17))
 (segment (start 122.7 89.3) (end 122.7 76.2) (width 0.2) (layer "F.Cu") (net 17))
 (via (at 131 37.3) (size 0.6) (drill 0.3) (layers "F.Cu" "B.Cu") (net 17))
 (segment (start 131 36.9) (end 134.5 33.4) (width 0.2) (layer "B.Cu") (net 17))
 (segment (start 131 37.3) (end 131 36.9) (width 0.2) (layer "B.Cu") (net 17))
 (segment (start 131.8 76) (end 131.8 31.1) (width 0.2) (layer "F.Cu") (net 16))
 (segment (start 130.7 76) (end 131.8 76) (width 0.2) (layer "F.Cu") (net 16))
 (segment (start 124.699 90.27863) (end 124.699 80.124) (width 0.2) (layer "F.Cu") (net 16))
 (segment (start 126.576 80.124) (end 130.7 76) (width 0.2) (layer "F.Cu") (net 16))
 (segment (start 116.9 97) (end 117.97763 97) (width 0.2) (layer "F.Cu") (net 16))
 (segment (start 131.8 31.1) (end 134.5 28.4) (width 0.2) (layer "F.Cu") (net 16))
 (segment (start 117.97763 97) (end 124.699 90.27863) (width 0.2) (layer "F.Cu") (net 16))
 (segment (start 124.699 80.124) (end 126.576 80.124) (width 0.2) (layer "F.Cu") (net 16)))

